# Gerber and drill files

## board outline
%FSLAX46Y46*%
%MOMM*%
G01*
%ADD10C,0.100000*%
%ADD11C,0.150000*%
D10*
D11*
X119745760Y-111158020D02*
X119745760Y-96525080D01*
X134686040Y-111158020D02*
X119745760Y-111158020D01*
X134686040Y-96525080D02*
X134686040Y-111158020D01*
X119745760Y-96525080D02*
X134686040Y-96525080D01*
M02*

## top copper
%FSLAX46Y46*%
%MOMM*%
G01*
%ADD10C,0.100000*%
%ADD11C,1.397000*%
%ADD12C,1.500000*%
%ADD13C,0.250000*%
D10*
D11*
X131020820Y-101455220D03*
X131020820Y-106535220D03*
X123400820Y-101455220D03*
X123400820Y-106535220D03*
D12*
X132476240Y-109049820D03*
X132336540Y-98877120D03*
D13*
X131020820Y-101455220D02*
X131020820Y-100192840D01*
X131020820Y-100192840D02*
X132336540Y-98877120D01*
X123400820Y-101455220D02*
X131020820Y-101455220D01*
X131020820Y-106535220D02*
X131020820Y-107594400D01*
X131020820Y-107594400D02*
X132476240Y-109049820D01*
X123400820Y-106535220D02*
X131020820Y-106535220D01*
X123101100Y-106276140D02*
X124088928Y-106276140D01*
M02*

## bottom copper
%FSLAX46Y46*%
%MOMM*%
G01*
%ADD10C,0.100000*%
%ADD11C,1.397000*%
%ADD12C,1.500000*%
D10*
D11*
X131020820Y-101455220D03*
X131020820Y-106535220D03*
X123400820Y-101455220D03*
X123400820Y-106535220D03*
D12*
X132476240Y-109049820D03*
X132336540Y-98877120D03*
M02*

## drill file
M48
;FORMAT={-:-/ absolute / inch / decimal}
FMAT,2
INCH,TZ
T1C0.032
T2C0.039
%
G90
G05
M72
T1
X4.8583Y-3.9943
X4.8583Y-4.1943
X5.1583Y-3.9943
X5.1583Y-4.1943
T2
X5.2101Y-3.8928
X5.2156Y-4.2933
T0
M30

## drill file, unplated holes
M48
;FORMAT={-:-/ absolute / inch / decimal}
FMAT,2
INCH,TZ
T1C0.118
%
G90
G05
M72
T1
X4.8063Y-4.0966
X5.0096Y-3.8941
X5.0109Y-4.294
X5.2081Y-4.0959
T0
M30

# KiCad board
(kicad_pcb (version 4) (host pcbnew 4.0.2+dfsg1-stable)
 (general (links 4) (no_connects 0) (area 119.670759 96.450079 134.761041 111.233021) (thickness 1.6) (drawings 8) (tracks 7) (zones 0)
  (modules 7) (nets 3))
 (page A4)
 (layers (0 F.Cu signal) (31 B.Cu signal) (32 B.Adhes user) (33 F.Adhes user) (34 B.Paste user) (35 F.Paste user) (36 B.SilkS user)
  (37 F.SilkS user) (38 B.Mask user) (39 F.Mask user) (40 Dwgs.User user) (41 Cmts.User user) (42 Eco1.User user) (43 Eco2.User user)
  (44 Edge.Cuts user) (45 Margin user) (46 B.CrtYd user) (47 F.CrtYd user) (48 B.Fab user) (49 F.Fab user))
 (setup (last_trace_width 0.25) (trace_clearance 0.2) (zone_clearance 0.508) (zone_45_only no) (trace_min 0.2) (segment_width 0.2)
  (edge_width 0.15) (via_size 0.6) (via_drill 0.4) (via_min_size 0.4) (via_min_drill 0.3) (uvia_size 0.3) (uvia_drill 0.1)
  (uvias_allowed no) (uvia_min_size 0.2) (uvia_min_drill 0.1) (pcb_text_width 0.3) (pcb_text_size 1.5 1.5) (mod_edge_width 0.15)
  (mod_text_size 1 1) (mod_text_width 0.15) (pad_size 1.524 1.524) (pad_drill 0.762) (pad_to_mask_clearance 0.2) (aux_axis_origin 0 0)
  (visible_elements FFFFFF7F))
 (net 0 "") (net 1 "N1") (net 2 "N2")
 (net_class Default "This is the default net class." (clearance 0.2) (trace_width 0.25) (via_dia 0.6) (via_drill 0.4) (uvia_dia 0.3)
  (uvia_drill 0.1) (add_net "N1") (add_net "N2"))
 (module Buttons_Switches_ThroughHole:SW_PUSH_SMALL (layer F.Cu) (at 127.21082 103.99522)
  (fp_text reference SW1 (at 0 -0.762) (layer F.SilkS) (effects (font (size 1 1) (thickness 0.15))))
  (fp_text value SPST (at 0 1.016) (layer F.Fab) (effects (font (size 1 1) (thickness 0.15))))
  (pad 1 thru_hole circle (at 3.81 -2.54) (size 1.397 1.397) (drill 0.8128) (layers *.Cu *.Mask F.SilkS) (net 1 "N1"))
  (pad 2 thru_hole circle (at 3.81 2.54) (size 1.397 1.397) (drill 0.8128) (layers *.Cu *.Mask F.SilkS) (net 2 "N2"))
  (pad 1 thru_hole circle (at -3.81 -2.54) (size 1.397 1.397) (drill 0.8128) (layers *.Cu *.Mask F.SilkS) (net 1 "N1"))
  (pad 2 thru_hole circle (at -3.81 2.54) (size 1.397 1.397) (drill 0.8128) (layers *.Cu *.Mask F.SilkS) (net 2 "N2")))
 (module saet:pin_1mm (layer F.Cu) (at 132.47624 109.04982)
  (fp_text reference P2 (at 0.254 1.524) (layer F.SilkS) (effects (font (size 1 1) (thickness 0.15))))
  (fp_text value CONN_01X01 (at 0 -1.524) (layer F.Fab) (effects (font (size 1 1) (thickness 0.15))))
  (pad 1 thru_hole circle (at 0 0) (size 1.5 1.5) (drill 1) (layers *.Cu *.Mask) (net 2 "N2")))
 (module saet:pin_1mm (layer F.Cu) (at 132.33654 98.87712)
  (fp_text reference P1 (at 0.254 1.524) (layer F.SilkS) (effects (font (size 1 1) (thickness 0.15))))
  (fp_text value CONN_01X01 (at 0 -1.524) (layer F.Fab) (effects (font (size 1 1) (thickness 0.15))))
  (pad 1 thru_hole circle (at 0 0) (size 1.5 1.5) (drill 1) (layers *.Cu *.Mask) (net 1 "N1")))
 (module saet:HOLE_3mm (layer F.Cu) (at 132.28574 104.03586)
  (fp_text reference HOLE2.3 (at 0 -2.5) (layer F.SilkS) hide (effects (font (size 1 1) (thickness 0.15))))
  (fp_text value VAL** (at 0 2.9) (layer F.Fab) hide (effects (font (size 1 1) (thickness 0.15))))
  (pad "" np_thru_hole circle (at 0 0) (size 3 3) (drill 3) (layers *.Cu *.Mask F.SilkS)))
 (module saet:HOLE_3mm (layer F.Cu) (at 127.24384 98.91014)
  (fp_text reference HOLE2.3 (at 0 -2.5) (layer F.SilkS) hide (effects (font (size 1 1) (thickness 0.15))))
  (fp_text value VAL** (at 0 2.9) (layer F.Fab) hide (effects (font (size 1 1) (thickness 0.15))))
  (pad "" np_thru_hole circle (at 0 0) (size 3 3) (drill 3) (layers *.Cu *.Mask F.SilkS)))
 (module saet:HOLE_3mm (layer F.Cu) (at 122.08002 104.05364)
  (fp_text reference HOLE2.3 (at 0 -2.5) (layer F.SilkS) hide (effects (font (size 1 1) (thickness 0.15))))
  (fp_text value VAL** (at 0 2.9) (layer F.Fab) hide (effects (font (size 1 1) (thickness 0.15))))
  (pad "" np_thru_hole circle (at 0 0) (size 3 3) (drill 3) (layers *.Cu *.Mask F.SilkS)))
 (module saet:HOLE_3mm (layer F.Cu) (at 127.27686 109.0676)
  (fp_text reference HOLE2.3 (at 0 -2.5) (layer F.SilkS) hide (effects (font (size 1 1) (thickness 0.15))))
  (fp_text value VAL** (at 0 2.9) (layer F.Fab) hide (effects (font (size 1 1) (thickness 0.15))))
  (pad "" np_thru_hole circle (at 0 0) (size 3 3) (drill 3) (layers *.Cu *.Mask F.SilkS)))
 (gr_line (start 119.74576 111.15802) (end 119.74576 96.52508) (layer Edge.Cuts) (width 0.15))
 (gr_line (start 134.68604 111.15802) (end 119.74576 111.15802) (layer Edge.Cuts) (width 0.15))
 (gr_line (start 134.68604 96.52508) (end 134.68604 111.15802) (layer Edge.Cuts) (width 0.15))
 (gr_line (start 119.74576 96.52508) (end 134.68604 96.52508) (layer Edge.Cuts) (width 0.15))
 (segment (start 131.02082 101.45522) (end 131.02082 100.19284) (width 0.25) (layer F.Cu) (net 1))
 (segment (start 131.02082 100.19284) (end 132.33654 98.87712) (width 0.25) (layer F.Cu) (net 1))
 (segment (start 123.40082 101.45522) (end 131.02082 101.45522) (width 0.25) (layer F.Cu) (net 1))
 (segment (start 131.02082 106.53522) (end 131.02082 107.5944) (width 0.25) (layer F.Cu) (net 2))
 (segment (start 131.02082 107.5944) (end 132.47624 109.04982) (width 0.25) (layer F.Cu) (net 2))
 (segment (start 123.40082 106.53522) (end 131.02082 106.53522) (width 0.25) (layer F.Cu) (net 2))
 (segment (start 123.1011 106.27614) (end 124.088928 106.27614) (width 0.25) (layer F.Cu) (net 2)))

